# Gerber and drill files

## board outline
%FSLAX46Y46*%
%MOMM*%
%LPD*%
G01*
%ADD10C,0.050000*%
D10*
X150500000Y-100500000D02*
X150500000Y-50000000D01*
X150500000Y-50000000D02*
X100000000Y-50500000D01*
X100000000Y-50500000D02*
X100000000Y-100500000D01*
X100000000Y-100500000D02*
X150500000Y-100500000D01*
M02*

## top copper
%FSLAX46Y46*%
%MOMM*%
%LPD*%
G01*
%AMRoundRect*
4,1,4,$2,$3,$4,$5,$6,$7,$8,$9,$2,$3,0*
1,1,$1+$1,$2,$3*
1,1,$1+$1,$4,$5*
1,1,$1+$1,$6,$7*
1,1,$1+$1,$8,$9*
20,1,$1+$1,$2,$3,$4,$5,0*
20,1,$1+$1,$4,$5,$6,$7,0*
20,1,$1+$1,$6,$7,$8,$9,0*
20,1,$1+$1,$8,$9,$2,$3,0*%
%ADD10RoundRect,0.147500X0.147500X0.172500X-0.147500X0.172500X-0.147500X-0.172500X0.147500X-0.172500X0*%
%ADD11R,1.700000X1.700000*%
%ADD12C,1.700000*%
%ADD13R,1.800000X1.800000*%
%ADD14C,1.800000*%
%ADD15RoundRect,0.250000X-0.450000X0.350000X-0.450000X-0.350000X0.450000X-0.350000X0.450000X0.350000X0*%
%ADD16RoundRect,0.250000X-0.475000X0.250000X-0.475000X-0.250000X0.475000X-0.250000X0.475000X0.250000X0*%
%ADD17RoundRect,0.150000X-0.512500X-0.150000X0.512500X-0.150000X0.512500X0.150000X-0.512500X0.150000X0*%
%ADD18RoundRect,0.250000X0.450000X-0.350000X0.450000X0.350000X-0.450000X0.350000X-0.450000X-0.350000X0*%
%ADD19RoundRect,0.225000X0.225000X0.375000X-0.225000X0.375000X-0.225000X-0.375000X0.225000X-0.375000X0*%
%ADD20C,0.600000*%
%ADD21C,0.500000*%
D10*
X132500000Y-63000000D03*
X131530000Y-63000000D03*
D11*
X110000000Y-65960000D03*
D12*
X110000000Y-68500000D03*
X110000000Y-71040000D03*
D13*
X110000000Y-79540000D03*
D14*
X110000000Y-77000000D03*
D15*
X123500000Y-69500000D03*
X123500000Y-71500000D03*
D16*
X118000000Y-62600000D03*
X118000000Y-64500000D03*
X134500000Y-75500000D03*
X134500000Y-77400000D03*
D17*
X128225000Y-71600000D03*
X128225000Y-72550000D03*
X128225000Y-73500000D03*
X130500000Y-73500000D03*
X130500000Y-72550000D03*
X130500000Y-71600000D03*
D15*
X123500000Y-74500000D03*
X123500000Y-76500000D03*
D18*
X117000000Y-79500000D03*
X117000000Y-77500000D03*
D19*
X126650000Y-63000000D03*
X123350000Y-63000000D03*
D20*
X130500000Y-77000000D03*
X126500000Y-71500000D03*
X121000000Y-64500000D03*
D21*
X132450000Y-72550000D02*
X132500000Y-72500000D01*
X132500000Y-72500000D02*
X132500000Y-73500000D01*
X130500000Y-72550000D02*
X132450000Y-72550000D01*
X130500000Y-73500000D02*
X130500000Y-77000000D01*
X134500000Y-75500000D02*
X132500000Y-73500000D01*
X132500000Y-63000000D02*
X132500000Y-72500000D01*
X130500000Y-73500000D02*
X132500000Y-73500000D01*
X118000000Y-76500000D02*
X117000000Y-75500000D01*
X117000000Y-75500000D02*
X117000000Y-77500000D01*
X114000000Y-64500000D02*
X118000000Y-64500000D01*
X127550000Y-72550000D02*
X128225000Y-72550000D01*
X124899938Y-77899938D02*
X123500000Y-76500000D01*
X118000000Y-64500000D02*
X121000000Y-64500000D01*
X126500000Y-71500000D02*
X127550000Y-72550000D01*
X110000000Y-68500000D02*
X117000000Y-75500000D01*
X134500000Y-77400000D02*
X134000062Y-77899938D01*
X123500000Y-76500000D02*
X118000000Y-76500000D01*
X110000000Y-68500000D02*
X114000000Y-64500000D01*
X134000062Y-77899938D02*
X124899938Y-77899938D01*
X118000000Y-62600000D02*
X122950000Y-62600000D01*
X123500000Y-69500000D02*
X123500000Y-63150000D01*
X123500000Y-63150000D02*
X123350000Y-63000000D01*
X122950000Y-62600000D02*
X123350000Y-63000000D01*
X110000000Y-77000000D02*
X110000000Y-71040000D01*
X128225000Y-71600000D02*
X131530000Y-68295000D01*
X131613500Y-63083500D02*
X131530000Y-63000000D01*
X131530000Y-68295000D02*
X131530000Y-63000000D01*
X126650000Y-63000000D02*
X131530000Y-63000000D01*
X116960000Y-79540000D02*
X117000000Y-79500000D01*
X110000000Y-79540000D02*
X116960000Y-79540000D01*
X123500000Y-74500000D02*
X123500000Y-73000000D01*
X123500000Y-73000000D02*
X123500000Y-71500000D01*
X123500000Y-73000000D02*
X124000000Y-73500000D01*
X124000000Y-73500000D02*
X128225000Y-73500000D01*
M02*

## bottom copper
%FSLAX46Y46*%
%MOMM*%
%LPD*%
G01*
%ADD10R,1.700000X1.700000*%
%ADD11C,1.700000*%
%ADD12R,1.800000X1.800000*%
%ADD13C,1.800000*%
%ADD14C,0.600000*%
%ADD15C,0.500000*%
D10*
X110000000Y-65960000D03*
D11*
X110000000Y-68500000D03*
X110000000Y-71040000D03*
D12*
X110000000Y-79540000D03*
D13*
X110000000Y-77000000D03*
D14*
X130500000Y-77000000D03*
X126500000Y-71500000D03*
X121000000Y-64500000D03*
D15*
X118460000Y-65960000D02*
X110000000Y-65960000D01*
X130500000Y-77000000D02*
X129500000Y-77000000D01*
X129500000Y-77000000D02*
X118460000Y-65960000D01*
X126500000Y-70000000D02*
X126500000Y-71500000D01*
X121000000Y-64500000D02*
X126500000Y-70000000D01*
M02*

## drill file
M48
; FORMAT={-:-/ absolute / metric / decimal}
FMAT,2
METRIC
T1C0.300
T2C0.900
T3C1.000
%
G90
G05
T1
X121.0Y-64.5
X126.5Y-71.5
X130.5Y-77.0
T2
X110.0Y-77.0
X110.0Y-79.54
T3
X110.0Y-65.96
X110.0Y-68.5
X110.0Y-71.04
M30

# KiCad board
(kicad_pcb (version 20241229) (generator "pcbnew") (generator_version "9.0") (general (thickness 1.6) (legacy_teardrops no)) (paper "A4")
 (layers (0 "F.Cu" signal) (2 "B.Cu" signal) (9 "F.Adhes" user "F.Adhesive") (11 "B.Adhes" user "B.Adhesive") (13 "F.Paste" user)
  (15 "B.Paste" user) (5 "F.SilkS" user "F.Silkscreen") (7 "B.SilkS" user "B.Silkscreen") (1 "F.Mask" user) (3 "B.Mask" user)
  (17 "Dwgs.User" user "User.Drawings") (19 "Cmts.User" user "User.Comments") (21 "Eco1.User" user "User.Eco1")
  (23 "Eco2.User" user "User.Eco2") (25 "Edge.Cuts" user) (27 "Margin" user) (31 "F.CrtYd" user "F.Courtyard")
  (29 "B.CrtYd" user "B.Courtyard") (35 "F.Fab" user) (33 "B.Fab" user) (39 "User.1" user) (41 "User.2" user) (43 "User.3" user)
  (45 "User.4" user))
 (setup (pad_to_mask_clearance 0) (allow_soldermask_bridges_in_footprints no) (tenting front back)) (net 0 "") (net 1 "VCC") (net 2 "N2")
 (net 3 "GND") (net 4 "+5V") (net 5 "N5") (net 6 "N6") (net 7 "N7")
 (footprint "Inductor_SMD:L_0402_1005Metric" (layer "F.Cu") (at 132.015 63 180)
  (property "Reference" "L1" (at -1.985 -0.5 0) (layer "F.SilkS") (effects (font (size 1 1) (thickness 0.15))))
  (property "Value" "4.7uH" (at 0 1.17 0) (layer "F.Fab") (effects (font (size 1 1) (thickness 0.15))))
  (pad "1" smd roundrect (at -0.485 0 180) (size 0.59 0.64) (layers "F.Cu" "F.Mask" "F.Paste") (roundrect_rratio 0.25) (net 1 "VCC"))
  (pad "2" smd roundrect (at 0.485 0 180) (size 0.59 0.64) (layers "F.Cu" "F.Mask" "F.Paste") (roundrect_rratio 0.25) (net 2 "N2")))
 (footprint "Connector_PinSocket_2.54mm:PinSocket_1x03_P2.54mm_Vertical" (layer "F.Cu") (at 110 65.96)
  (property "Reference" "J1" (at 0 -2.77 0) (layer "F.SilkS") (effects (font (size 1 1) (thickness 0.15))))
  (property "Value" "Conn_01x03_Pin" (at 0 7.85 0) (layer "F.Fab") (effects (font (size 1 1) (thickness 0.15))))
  (pad "1" thru_hole rect (at 0 0) (size 1.7 1.7) (drill 1) (layers "*.Cu" "*.Mask") (remove_unused_layers no) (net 1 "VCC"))
  (pad "2" thru_hole circle (at 0 2.54) (size 1.7 1.7) (drill 1) (layers "*.Cu" "*.Mask") (remove_unused_layers no) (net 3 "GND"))
  (pad "3" thru_hole circle (at 0 5.08) (size 1.7 1.7) (drill 1) (layers "*.Cu" "*.Mask") (remove_unused_layers no) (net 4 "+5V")))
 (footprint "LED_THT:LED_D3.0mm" (layer "F.Cu") (at 110 79.54 90)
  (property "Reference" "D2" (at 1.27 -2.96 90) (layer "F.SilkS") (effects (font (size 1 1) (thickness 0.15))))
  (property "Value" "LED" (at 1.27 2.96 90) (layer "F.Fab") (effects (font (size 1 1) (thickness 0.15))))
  (pad "1" thru_hole rect (at 0 0 90) (size 1.8 1.8) (drill 0.9) (layers "*.Cu" "*.Mask") (remove_unused_layers no) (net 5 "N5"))
  (pad "2" thru_hole circle (at 2.54 0 90) (size 1.8 1.8) (drill 0.9) (layers "*.Cu" "*.Mask") (remove_unused_layers no) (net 4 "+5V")))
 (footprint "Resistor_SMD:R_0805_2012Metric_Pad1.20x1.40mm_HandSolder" (layer "F.Cu") (at 123.5 70.5 -90)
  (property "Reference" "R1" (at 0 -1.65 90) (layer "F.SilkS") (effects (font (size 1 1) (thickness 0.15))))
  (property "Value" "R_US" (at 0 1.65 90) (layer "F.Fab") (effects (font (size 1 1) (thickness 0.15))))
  (pad "1" smd roundrect (at -1 0 270) (size 1.2 1.4) (layers "F.Cu" "F.Mask" "F.Paste") (roundrect_rratio 0.208333) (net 4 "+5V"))
  (pad "2" smd roundrect (at 1 0 270) (size 1.2 1.4) (layers "F.Cu" "F.Mask" "F.Paste") (roundrect_rratio 0.208333) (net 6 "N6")))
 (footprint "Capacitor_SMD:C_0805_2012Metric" (layer "F.Cu") (at 118 63.55 -90)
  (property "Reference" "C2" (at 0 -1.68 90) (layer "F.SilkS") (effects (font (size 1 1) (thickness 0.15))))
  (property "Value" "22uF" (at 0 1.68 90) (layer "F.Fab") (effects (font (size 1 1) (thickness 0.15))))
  (pad "1" smd roundrect (at -0.95 0 270) (size 1 1.45) (layers "F.Cu" "F.Mask" "F.Paste") (roundrect_rratio 0.25) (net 4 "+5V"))
  (pad "2" smd roundrect (at 0.95 0 270) (size 1 1.45) (layers "F.Cu" "F.Mask" "F.Paste") (roundrect_rratio 0.25) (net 3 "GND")))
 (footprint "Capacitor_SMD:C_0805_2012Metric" (layer "F.Cu") (at 134.5 76.45 -90)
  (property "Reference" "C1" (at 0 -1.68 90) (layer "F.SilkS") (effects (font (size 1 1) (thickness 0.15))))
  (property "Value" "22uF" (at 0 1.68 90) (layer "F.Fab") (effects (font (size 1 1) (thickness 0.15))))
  (pad "1" smd roundrect (at -0.95 0 270) (size 1 1.45) (layers "F.Cu" "F.Mask" "F.Paste") (roundrect_rratio 0.25) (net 1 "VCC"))
  (pad "2" smd roundrect (at 0.95 0 270) (size 1 1.45) (layers "F.Cu" "F.Mask" "F.Paste") (roundrect_rratio 0.25) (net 3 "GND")))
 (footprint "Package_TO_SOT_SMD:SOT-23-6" (layer "F.Cu") (at 129.3625 72.55)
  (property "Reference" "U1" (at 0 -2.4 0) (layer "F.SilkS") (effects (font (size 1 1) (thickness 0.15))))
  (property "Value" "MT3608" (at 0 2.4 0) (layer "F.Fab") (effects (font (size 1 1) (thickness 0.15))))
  (pad "1" smd roundrect (at -1.1375 -0.95) (size 1.325 0.6) (layers "F.Cu" "F.Mask" "F.Paste") (roundrect_rratio 0.25) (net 2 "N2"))
  (pad "2" smd roundrect (at -1.1375 0) (size 1.325 0.6) (layers "F.Cu" "F.Mask" "F.Paste") (roundrect_rratio 0.25) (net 3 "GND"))
  (pad "3" smd roundrect (at -1.1375 0.95) (size 1.325 0.6) (layers "F.Cu" "F.Mask" "F.Paste") (roundrect_rratio 0.25) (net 6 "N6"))
  (pad "4" smd roundrect (at 1.1375 0.95) (size 1.325 0.6) (layers "F.Cu" "F.Mask" "F.Paste") (roundrect_rratio 0.25) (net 1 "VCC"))
  (pad "5" smd roundrect (at 1.1375 0) (size 1.325 0.6) (layers "F.Cu" "F.Mask" "F.Paste") (roundrect_rratio 0.25) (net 1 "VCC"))
  (pad "6" smd roundrect (at 1.1375 -0.95) (size 1.325 0.6) (layers "F.Cu" "F.Mask" "F.Paste") (roundrect_rratio 0.25) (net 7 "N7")))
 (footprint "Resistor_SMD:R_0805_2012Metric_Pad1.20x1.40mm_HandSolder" (layer "F.Cu") (at 123.5 75.5 -90)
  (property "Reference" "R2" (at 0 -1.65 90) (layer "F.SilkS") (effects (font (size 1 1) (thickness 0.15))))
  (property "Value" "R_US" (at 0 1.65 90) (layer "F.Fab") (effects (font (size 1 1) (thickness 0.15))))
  (pad "1" smd roundrect (at -1 0 270) (size 1.2 1.4) (layers "F.Cu" "F.Mask" "F.Paste") (roundrect_rratio 0.208333) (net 6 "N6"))
  (pad "2" smd roundrect (at 1 0 270) (size 1.2 1.4) (layers "F.Cu" "F.Mask" "F.Paste") (roundrect_rratio 0.208333) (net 3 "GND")))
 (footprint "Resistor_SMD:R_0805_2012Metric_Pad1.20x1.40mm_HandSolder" (layer "F.Cu") (at 117 78.5 90)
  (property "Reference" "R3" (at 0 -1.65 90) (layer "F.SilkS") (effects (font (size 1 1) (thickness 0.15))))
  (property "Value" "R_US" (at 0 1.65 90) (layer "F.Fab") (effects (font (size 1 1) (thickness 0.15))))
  (pad "1" smd roundrect (at -1 0 90) (size 1.2 1.4) (layers "F.Cu" "F.Mask" "F.Paste") (roundrect_rratio 0.208333) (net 5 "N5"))
  (pad "2" smd roundrect (at 1 0 90) (size 1.2 1.4) (layers "F.Cu" "F.Mask" "F.Paste") (roundrect_rratio 0.208333) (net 3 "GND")))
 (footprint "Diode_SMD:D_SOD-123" (layer "F.Cu") (at 125 63 180)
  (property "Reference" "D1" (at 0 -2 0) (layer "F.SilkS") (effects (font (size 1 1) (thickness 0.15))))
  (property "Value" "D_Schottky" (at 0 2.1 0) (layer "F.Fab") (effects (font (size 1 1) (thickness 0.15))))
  (pad "1" smd roundrect (at -1.65 0 180) (size 0.9 1.2) (layers "F.Cu" "F.Mask" "F.Paste") (roundrect_rratio 0.25) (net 2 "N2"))
  (pad "2" smd roundrect (at 1.65 0 180) (size 0.9 1.2) (layers "F.Cu" "F.Mask" "F.Paste") (roundrect_rratio 0.25) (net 4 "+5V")))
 (gr_line (start 150.5 100.5) (end 150.5 50) (stroke (width 0.05) (type default)) (layer "Edge.Cuts"))
 (gr_line (start 150.5 50) (end 100 50.5) (stroke (width 0.05) (type default)) (layer "Edge.Cuts"))
 (gr_line (start 100 50.5) (end 100 100.5) (stroke (width 0.05) (type default)) (layer "Edge.Cuts"))
 (gr_line (start 100 100.5) (end 150.5 100.5) (stroke (width 0.05) (type default)) (layer "Edge.Cuts"))
 (segment (start 132.45 72.55) (end 132.5 72.5) (width 0.5) (layer "F.Cu") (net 1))
 (segment (start 132.5 72.5) (end 132.5 73.5) (width 0.5) (layer "F.Cu") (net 1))
 (segment (start 130.5 72.55) (end 132.45 72.55) (width 0.5) (layer "F.Cu") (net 1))
 (segment (start 130.5 73.5) (end 130.5 77) (width 0.5) (layer "F.Cu") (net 1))
 (segment (start 134.5 75.5) (end 132.5 73.5) (width 0.5) (layer "F.Cu") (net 1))
 (segment (start 132.5 63) (end 132.5 72.5) (width 0.5) (layer "F.Cu") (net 1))
 (segment (start 130.5 73.5) (end 132.5 73.5) (width 0.5) (layer "F.Cu") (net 1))
 (via (at 130.5 77) (size 0.6) (drill 0.3) (layers "F.Cu" "B.Cu") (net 1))
 (segment (start 118.46 65.96) (end 110 65.96) (width 0.5) (layer "B.Cu") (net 1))
 (segment (start 130.5 77) (end 129.5 77) (width 0.5) (layer "B.Cu") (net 1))
 (segment (start 129.5 77) (end 118.46 65.96) (width 0.5) (layer "B.Cu") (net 1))
 (segment (start 118 76.5) (end 117 75.5) (width 0.5) (layer "F.Cu") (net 3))
 (segment (start 117 75.5) (end 117 77.5) (width 0.5) (layer "F.Cu") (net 3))
 (segment (start 114 64.5) (end 118 64.5) (width 0.5) (layer "F.Cu") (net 3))
 (segment (start 127.55 72.55) (end 128.225 72.55) (width 0.5) (layer "F.Cu") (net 3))
 (segment (start 124.899938 77.899938) (end 123.5 76.5) (width 0.5) (layer "F.Cu") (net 3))
 (segment (start 118 64.5) (end 121 64.5) (width 0.5) (layer "F.Cu") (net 3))
 (segment (start 126.5 71.5) (end 127.55 72.55) (width 0.5) (layer "F.Cu") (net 3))
 (segment (start 110 68.5) (end 117 75.5) (width 0.5) (layer "F.Cu") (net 3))
 (segment (start 134.5 77.4) (end 134.000062 77.899938) (width 0.5) (layer "F.Cu") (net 3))
 (segment (start 123.5 76.5) (end 118 76.5) (width 0.5) (layer "F.Cu") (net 3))
 (segment (start 110 68.5) (end 114 64.5) (width 0.5) (layer "F.Cu") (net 3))
 (segment (start 134.000062 77.899938) (end 124.899938 77.899938) (width 0.5) (layer "F.Cu") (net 3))
 (via (at 126.5 71.5) (size 0.6) (drill 0.3) (layers "F.Cu" "B.Cu") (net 3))
 (via (at 121 64.5) (size 0.6) (drill 0.3) (layers "F.Cu" "B.Cu") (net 3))
 (segment (start 126.5 70) (end 126.5 71.5) (width 0.5) (layer "B.Cu") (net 3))
 (segment (start 121 64.5) (end 126.5 70) (width 0.5) (layer "B.Cu") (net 3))
 (segment (start 118 62.6) (end 122.95 62.6) (width 0.5) (layer "F.Cu") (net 4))
 (segment (start 123.5 69.5) (end 123.5 63.15) (width 0.5) (layer "F.Cu") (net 4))
 (segment (start 123.5 63.15) (end 123.35 63) (width 0.5) (layer "F.Cu") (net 4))
 (segment (start 122.95 62.6) (end 123.35 63) (width 0.5) (layer "F.Cu") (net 4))
 (segment (start 110 77) (end 110 71.04) (width 0.5) (layer "F.Cu") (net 4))
 (segment (start 128.225 71.6) (end 131.53 68.295) (width 0.5) (layer "F.Cu") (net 2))
 (segment (start 131.6135 63.0835) (end 131.53 63) (width 0.5) (layer "F.Cu") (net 2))
 (segment (start 131.53 68.295) (end 131.53 63) (width 0.5) (layer "F.Cu") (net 2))
 (segment (start 126.65 63) (end 131.53 63) (width 0.5) (layer "F.Cu") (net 2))
 (segment (start 116.96 79.54) (end 117 79.5) (width 0.5) (layer "F.Cu") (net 5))
 (segment (start 110 79.54) (end 116.96 79.54) (width 0.5) (layer "F.Cu") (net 5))
 (segment (start 123.5 74.5) (end 123.5 73) (width 0.5) (layer "F.Cu") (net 6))
 (segment (start 123.5 73) (end 123.5 71.5) (width 0.5) (layer "F.Cu") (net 6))
 (segment (start 123.5 73) (end 124 73.5) (width 0.5) (layer "F.Cu") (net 6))
 (segment (start 124 73.5) (end 128.225 73.5) (width 0.5) (layer "F.Cu") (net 6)))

